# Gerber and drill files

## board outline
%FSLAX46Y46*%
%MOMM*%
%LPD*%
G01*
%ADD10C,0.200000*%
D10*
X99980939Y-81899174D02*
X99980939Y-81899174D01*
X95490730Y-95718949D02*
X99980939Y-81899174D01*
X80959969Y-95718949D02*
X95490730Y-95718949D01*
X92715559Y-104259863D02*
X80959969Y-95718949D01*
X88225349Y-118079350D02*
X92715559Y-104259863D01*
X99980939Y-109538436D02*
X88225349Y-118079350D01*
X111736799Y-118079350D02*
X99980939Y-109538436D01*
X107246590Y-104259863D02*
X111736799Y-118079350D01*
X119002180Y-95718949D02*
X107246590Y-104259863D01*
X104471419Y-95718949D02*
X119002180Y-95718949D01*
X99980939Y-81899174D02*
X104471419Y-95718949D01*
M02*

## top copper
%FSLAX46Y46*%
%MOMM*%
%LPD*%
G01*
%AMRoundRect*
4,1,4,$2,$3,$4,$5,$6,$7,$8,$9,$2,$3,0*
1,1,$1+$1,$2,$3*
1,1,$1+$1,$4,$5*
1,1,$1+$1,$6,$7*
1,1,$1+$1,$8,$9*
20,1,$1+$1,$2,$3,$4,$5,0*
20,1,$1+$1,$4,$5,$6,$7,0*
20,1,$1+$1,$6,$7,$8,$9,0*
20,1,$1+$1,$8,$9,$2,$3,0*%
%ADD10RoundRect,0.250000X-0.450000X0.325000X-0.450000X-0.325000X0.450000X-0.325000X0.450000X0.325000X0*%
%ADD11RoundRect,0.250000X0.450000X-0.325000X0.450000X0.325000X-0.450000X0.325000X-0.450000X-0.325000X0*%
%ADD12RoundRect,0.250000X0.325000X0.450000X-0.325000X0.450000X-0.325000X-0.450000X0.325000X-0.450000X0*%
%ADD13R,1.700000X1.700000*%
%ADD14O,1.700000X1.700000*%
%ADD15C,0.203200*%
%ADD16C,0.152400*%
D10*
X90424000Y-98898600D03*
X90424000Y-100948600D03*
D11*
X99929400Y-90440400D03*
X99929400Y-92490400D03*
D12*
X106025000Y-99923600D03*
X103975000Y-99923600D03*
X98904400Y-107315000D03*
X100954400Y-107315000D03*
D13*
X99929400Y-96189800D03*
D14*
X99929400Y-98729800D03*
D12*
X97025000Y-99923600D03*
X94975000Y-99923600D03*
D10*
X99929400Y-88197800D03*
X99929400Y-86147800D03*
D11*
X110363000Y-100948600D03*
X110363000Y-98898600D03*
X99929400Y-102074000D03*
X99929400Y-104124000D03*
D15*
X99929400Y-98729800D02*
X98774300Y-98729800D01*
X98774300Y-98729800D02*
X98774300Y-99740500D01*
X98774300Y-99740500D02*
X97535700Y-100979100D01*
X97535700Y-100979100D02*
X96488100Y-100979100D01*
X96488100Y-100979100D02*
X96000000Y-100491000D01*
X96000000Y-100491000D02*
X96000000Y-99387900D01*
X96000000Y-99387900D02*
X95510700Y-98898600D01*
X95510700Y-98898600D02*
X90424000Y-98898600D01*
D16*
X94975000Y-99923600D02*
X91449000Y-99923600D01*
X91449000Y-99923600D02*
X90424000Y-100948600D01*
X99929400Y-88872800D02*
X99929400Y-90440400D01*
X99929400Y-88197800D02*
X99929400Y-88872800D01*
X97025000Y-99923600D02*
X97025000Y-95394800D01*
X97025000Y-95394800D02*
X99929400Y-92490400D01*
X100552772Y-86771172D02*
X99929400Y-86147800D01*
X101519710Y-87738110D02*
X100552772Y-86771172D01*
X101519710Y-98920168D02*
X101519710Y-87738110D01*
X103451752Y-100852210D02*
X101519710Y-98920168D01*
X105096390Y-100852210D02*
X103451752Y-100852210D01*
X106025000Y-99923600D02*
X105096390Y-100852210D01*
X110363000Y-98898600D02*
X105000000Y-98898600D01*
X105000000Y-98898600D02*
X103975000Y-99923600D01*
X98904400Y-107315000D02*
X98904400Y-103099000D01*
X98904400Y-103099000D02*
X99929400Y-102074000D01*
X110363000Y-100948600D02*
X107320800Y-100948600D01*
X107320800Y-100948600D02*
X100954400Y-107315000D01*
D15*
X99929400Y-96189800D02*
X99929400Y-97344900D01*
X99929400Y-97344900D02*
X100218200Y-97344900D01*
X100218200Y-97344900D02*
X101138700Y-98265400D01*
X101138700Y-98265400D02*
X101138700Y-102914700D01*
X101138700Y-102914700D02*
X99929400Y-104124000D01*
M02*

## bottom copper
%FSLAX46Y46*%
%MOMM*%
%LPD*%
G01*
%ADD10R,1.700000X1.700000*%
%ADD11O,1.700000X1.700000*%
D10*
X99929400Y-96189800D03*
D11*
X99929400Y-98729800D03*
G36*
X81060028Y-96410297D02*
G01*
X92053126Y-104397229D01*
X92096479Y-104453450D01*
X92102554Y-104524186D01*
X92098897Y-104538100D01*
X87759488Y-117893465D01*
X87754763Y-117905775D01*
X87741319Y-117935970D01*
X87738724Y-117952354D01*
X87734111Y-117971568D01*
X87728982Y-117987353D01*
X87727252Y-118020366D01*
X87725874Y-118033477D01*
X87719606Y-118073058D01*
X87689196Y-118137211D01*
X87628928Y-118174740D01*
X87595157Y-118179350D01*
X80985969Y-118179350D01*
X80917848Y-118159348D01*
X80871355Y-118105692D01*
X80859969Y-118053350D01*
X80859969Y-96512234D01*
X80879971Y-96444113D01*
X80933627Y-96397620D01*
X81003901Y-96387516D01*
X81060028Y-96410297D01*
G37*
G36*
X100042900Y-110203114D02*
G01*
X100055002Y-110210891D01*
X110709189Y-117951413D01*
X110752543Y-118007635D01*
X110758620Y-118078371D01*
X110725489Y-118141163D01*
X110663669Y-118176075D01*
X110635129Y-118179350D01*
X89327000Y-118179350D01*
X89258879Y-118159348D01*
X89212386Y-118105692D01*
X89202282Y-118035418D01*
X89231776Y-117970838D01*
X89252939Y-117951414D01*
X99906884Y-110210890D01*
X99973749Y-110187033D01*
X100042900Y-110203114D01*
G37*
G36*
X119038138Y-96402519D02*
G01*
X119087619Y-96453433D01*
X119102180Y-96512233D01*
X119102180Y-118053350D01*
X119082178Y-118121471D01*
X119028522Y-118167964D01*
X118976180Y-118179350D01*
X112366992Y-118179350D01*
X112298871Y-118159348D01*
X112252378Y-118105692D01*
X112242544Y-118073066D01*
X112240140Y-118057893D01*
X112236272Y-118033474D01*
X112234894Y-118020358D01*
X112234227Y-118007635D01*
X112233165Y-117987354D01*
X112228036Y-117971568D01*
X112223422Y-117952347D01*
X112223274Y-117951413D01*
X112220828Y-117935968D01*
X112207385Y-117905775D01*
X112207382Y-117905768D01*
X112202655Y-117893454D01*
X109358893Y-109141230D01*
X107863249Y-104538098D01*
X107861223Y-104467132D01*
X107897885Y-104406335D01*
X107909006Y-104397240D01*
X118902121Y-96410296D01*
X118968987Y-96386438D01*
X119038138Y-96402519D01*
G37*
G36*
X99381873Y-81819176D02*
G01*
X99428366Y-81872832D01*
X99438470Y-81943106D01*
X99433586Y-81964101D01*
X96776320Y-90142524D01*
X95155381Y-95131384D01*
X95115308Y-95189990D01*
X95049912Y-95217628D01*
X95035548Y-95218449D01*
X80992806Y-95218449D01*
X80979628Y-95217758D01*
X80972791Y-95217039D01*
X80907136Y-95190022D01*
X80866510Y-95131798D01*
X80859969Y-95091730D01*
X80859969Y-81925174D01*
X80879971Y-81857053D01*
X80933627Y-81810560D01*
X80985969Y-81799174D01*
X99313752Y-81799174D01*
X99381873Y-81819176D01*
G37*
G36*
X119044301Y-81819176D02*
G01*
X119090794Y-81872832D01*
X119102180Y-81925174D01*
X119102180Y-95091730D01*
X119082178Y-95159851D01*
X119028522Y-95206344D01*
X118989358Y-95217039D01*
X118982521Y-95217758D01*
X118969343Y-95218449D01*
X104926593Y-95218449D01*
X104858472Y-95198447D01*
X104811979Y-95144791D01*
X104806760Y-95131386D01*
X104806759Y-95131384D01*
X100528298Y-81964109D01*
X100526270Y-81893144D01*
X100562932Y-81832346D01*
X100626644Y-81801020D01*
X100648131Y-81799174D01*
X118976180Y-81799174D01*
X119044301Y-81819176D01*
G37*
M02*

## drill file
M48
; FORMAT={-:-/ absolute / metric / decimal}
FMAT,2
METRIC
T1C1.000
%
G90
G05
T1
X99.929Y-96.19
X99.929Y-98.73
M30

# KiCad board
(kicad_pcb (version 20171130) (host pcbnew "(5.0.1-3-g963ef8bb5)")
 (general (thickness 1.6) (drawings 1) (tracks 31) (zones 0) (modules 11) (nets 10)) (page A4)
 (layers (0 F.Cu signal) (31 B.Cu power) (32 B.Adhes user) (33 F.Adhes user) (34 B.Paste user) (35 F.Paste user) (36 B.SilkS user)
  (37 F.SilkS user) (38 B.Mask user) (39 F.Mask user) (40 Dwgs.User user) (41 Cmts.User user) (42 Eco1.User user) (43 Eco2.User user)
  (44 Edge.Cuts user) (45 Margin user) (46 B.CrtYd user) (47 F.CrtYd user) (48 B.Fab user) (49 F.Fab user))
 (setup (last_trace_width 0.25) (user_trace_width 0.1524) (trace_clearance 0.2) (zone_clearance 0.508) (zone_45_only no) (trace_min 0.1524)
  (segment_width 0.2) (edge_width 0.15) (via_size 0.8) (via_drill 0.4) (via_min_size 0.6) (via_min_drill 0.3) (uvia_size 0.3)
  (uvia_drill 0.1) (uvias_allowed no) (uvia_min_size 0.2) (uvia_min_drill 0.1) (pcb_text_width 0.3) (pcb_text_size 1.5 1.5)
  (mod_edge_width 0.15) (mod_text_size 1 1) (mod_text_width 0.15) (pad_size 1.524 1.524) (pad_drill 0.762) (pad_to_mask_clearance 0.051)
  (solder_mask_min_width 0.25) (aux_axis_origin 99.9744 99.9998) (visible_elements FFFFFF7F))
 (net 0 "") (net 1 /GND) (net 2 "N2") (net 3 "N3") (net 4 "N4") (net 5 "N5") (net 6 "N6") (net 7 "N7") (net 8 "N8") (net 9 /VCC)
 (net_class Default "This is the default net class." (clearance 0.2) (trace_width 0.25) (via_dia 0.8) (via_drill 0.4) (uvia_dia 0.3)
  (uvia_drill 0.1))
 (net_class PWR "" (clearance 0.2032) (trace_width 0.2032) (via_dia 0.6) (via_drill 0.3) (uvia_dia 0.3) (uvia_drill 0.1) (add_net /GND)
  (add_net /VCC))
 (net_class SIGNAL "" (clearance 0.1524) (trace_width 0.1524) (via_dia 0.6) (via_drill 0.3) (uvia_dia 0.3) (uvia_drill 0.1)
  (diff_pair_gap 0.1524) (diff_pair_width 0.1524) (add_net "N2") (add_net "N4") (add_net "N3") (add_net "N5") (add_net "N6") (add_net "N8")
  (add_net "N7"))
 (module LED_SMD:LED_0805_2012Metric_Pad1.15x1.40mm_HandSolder (layer F.Cu) (at 90.424 99.9236 270)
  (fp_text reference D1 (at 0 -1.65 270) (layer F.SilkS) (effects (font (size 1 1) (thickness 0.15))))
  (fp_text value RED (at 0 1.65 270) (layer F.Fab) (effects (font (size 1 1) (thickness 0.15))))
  (pad 1 smd roundrect (at -1.025 0 270) (size 1.15 1.4) (layers F.Cu F.Paste F.Mask) (roundrect_rratio 0.217391) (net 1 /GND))
  (pad 2 smd roundrect (at 1.025 0 270) (size 1.15 1.4) (layers F.Cu F.Paste F.Mask) (roundrect_rratio 0.217391) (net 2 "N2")))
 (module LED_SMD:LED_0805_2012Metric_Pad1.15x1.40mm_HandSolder (layer F.Cu) (at 99.9294 91.4654 90)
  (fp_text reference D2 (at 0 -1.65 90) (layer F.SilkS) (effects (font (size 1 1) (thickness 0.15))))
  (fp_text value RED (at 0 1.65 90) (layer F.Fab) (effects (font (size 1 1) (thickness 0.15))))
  (pad 2 smd roundrect (at 1.025 0 90) (size 1.15 1.4) (layers F.Cu F.Paste F.Mask) (roundrect_rratio 0.217391) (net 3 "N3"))
  (pad 1 smd roundrect (at -1.025 0 90) (size 1.15 1.4) (layers F.Cu F.Paste F.Mask) (roundrect_rratio 0.217391) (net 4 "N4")))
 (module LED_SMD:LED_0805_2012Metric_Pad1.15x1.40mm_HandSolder (layer F.Cu) (at 105 99.9236 180)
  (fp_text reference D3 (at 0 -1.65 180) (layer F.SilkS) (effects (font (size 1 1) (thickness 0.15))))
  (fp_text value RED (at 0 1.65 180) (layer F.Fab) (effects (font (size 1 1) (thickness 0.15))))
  (pad 1 smd roundrect (at -1.025 0 180) (size 1.15 1.4) (layers F.Cu F.Paste F.Mask) (roundrect_rratio 0.217391) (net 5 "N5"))
  (pad 2 smd roundrect (at 1.025 0 180) (size 1.15 1.4) (layers F.Cu F.Paste F.Mask) (roundrect_rratio 0.217391) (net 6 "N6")))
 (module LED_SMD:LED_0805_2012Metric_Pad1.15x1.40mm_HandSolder (layer F.Cu) (at 99.9294 107.315 180)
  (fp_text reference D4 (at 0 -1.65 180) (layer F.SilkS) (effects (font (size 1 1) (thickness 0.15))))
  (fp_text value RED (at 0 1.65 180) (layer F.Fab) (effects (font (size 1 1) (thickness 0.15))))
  (pad 2 smd roundrect (at 1.025 0 180) (size 1.15 1.4) (layers F.Cu F.Paste F.Mask) (roundrect_rratio 0.217391) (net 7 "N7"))
  (pad 1 smd roundrect (at -1.025 0 180) (size 1.15 1.4) (layers F.Cu F.Paste F.Mask) (roundrect_rratio 0.217391) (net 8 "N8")))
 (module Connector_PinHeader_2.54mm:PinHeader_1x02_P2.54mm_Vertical (layer F.Cu) (at 99.9294 96.1898)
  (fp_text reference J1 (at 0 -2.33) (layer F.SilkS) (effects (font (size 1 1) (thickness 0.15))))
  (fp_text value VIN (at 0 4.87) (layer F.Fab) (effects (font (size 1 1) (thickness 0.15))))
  (pad 1 thru_hole rect (at 0 0) (size 1.7 1.7) (drill 1) (layers *.Cu *.Mask) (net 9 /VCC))
  (pad 2 thru_hole oval (at 0 2.54) (size 1.7 1.7) (drill 1) (layers *.Cu *.Mask) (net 1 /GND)))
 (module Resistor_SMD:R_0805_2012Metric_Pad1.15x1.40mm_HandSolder (layer F.Cu) (at 96 99.9236 180)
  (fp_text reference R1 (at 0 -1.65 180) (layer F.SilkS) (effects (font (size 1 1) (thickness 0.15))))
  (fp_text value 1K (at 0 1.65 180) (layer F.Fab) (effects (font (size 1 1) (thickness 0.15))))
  (pad 1 smd roundrect (at -1.025 0 180) (size 1.15 1.4) (layers F.Cu F.Paste F.Mask) (roundrect_rratio 0.217391) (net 4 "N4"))
  (pad 2 smd roundrect (at 1.025 0 180) (size 1.15 1.4) (layers F.Cu F.Paste F.Mask) (roundrect_rratio 0.217391) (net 2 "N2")))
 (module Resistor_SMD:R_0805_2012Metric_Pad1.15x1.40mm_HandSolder (layer F.Cu) (at 99.9294 87.1728 270)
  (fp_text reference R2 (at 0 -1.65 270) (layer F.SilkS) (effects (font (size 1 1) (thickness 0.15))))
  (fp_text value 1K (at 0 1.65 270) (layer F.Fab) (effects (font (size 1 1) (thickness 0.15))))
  (pad 2 smd roundrect (at 1.025 0 270) (size 1.15 1.4) (layers F.Cu F.Paste F.Mask) (roundrect_rratio 0.217391) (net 3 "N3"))
  (pad 1 smd roundrect (at -1.025 0 270) (size 1.15 1.4) (layers F.Cu F.Paste F.Mask) (roundrect_rratio 0.217391) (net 5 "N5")))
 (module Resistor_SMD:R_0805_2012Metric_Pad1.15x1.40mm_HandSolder (layer F.Cu) (at 110.363 99.9236 90)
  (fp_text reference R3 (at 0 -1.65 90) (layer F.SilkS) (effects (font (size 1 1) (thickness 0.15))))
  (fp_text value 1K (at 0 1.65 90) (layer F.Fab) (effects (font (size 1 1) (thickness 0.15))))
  (pad 1 smd roundrect (at -1.025 0 90) (size 1.15 1.4) (layers F.Cu F.Paste F.Mask) (roundrect_rratio 0.217391) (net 8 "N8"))
  (pad 2 smd roundrect (at 1.025 0 90) (size 1.15 1.4) (layers F.Cu F.Paste F.Mask) (roundrect_rratio 0.217391) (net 6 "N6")))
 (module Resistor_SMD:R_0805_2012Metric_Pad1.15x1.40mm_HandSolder (layer F.Cu) (at 99.9294 103.099 90)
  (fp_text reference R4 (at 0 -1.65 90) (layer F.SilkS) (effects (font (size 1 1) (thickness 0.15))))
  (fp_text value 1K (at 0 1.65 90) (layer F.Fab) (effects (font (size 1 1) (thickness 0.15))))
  (pad 2 smd roundrect (at 1.025 0 90) (size 1.15 1.4) (layers F.Cu F.Paste F.Mask) (roundrect_rratio 0.217391) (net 7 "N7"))
  (pad 1 smd roundrect (at -1.025 0 90) (size 1.15 1.4) (layers F.Cu F.Paste F.Mask) (roundrect_rratio 0.217391) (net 9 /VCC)))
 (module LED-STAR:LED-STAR (layer F.Cu) (at 100 100)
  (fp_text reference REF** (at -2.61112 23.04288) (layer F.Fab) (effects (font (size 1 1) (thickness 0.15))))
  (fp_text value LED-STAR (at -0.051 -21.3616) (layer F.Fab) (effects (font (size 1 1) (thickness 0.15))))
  (fp_line (start -0.019061 -18.100826) (end -0.019061 -18.100826) (layer Edge.Cuts) (width 0.2))
  (fp_line (start -4.50927 -4.281051) (end -0.019061 -18.100826) (layer Edge.Cuts) (width 0.2))
  (fp_line (start -19.040031 -4.281051) (end -4.50927 -4.281051) (layer Edge.Cuts) (width 0.2))
  (fp_line (start -7.284441 4.259863) (end -19.040031 -4.281051) (layer Edge.Cuts) (width 0.2))
  (fp_line (start -11.774651 18.07935) (end -7.284441 4.259863) (layer Edge.Cuts) (width 0.2))
  (fp_line (start -0.019061 9.538436) (end -11.774651 18.07935) (layer Edge.Cuts) (width 0.2))
  (fp_line (start 11.736799 18.07935) (end -0.019061 9.538436) (layer Edge.Cuts) (width 0.2))
  (fp_line (start 7.24659 4.259863) (end 11.736799 18.07935) (layer Edge.Cuts) (width 0.2))
  (fp_line (start 19.00218 -4.281051) (end 7.24659 4.259863) (layer Edge.Cuts) (width 0.2))
  (fp_line (start 4.471419 -4.281051) (end 19.00218 -4.281051) (layer Edge.Cuts) (width 0.2))
  (fp_line (start -0.019061 -18.100826) (end 4.471419 -4.281051) (layer Edge.Cuts) (width 0.2)))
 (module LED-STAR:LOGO (layer B.Cu) (at 99.4029 102.9716 180)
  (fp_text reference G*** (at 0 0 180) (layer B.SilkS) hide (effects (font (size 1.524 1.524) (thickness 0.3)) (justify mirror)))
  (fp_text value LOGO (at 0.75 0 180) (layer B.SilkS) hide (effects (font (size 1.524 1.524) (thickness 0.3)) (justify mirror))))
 (segment (start 99.9294 98.7298) (end 98.7743 98.7298) (width 0.2032) (layer F.Cu) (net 1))
 (segment (start 98.7743 98.7298) (end 98.7743 99.7405) (width 0.2032) (layer F.Cu) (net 1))
 (segment (start 98.7743 99.7405) (end 97.5357 100.9791) (width 0.2032) (layer F.Cu) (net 1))
 (segment (start 97.5357 100.9791) (end 96.4881 100.9791) (width 0.2032) (layer F.Cu) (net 1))
 (segment (start 96.4881 100.9791) (end 96 100.491) (width 0.2032) (layer F.Cu) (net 1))
 (segment (start 96 100.491) (end 96 99.3879) (width 0.2032) (layer F.Cu) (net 1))
 (segment (start 96 99.3879) (end 95.5107 98.8986) (width 0.2032) (layer F.Cu) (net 1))
 (segment (start 95.5107 98.8986) (end 90.424 98.8986) (width 0.2032) (layer F.Cu) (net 1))
 (segment (start 94.975 99.9236) (end 91.449 99.9236) (width 0.1524) (layer F.Cu) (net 2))
 (segment (start 91.449 99.9236) (end 90.424 100.9486) (width 0.1524) (layer F.Cu) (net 2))
 (segment (start 99.9294 88.8728) (end 99.9294 90.4404) (width 0.1524) (layer F.Cu) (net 3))
 (segment (start 99.9294 88.1978) (end 99.9294 88.8728) (width 0.1524) (layer F.Cu) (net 3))
 (segment (start 97.025 99.9236) (end 97.025 95.3948) (width 0.1524) (layer F.Cu) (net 4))
 (segment (start 97.025 95.3948) (end 99.9294 92.4904) (width 0.1524) (layer F.Cu) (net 4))
 (segment (start 100.552772 86.771172) (end 99.9294 86.1478) (width 0.1524) (layer F.Cu) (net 5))
 (segment (start 101.51971 87.73811) (end 100.552772 86.771172) (width 0.1524) (layer F.Cu) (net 5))
 (segment (start 101.51971 98.920168) (end 101.51971 87.73811) (width 0.1524) (layer F.Cu) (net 5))
 (segment (start 103.451752 100.85221) (end 101.51971 98.920168) (width 0.1524) (layer F.Cu) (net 5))
 (segment (start 105.09639 100.85221) (end 103.451752 100.85221) (width 0.1524) (layer F.Cu) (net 5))
 (segment (start 106.025 99.9236) (end 105.09639 100.85221) (width 0.1524) (layer F.Cu) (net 5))
 (segment (start 110.363 98.8986) (end 105 98.8986) (width 0.1524) (layer F.Cu) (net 6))
 (segment (start 105 98.8986) (end 103.975 99.9236) (width 0.1524) (layer F.Cu) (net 6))
 (segment (start 98.9044 107.315) (end 98.9044 103.099) (width 0.1524) (layer F.Cu) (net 7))
 (segment (start 98.9044 103.099) (end 99.9294 102.074) (width 0.1524) (layer F.Cu) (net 7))
 (segment (start 110.363 100.9486) (end 107.3208 100.9486) (width 0.1524) (layer F.Cu) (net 8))
 (segment (start 107.3208 100.9486) (end 100.9544 107.315) (width 0.1524) (layer F.Cu) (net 8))
 (segment (start 99.9294 96.1898) (end 99.9294 97.3449) (width 0.2032) (layer F.Cu) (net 9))
 (segment (start 99.9294 97.3449) (end 100.2182 97.3449) (width 0.2032) (layer F.Cu) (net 9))
 (segment (start 100.2182 97.3449) (end 101.1387 98.2654) (width 0.2032) (layer F.Cu) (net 9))
 (segment (start 101.1387 98.2654) (end 101.1387 102.9147) (width 0.2032) (layer F.Cu) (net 9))
 (segment (start 101.1387 102.9147) (end 99.9294 104.124) (width 0.2032) (layer F.Cu) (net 9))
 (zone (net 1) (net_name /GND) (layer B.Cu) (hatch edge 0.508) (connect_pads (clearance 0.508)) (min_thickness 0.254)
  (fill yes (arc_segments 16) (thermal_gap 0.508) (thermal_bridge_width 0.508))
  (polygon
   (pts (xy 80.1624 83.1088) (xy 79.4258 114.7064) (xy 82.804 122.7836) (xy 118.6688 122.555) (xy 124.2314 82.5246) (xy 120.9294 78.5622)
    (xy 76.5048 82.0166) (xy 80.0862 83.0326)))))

